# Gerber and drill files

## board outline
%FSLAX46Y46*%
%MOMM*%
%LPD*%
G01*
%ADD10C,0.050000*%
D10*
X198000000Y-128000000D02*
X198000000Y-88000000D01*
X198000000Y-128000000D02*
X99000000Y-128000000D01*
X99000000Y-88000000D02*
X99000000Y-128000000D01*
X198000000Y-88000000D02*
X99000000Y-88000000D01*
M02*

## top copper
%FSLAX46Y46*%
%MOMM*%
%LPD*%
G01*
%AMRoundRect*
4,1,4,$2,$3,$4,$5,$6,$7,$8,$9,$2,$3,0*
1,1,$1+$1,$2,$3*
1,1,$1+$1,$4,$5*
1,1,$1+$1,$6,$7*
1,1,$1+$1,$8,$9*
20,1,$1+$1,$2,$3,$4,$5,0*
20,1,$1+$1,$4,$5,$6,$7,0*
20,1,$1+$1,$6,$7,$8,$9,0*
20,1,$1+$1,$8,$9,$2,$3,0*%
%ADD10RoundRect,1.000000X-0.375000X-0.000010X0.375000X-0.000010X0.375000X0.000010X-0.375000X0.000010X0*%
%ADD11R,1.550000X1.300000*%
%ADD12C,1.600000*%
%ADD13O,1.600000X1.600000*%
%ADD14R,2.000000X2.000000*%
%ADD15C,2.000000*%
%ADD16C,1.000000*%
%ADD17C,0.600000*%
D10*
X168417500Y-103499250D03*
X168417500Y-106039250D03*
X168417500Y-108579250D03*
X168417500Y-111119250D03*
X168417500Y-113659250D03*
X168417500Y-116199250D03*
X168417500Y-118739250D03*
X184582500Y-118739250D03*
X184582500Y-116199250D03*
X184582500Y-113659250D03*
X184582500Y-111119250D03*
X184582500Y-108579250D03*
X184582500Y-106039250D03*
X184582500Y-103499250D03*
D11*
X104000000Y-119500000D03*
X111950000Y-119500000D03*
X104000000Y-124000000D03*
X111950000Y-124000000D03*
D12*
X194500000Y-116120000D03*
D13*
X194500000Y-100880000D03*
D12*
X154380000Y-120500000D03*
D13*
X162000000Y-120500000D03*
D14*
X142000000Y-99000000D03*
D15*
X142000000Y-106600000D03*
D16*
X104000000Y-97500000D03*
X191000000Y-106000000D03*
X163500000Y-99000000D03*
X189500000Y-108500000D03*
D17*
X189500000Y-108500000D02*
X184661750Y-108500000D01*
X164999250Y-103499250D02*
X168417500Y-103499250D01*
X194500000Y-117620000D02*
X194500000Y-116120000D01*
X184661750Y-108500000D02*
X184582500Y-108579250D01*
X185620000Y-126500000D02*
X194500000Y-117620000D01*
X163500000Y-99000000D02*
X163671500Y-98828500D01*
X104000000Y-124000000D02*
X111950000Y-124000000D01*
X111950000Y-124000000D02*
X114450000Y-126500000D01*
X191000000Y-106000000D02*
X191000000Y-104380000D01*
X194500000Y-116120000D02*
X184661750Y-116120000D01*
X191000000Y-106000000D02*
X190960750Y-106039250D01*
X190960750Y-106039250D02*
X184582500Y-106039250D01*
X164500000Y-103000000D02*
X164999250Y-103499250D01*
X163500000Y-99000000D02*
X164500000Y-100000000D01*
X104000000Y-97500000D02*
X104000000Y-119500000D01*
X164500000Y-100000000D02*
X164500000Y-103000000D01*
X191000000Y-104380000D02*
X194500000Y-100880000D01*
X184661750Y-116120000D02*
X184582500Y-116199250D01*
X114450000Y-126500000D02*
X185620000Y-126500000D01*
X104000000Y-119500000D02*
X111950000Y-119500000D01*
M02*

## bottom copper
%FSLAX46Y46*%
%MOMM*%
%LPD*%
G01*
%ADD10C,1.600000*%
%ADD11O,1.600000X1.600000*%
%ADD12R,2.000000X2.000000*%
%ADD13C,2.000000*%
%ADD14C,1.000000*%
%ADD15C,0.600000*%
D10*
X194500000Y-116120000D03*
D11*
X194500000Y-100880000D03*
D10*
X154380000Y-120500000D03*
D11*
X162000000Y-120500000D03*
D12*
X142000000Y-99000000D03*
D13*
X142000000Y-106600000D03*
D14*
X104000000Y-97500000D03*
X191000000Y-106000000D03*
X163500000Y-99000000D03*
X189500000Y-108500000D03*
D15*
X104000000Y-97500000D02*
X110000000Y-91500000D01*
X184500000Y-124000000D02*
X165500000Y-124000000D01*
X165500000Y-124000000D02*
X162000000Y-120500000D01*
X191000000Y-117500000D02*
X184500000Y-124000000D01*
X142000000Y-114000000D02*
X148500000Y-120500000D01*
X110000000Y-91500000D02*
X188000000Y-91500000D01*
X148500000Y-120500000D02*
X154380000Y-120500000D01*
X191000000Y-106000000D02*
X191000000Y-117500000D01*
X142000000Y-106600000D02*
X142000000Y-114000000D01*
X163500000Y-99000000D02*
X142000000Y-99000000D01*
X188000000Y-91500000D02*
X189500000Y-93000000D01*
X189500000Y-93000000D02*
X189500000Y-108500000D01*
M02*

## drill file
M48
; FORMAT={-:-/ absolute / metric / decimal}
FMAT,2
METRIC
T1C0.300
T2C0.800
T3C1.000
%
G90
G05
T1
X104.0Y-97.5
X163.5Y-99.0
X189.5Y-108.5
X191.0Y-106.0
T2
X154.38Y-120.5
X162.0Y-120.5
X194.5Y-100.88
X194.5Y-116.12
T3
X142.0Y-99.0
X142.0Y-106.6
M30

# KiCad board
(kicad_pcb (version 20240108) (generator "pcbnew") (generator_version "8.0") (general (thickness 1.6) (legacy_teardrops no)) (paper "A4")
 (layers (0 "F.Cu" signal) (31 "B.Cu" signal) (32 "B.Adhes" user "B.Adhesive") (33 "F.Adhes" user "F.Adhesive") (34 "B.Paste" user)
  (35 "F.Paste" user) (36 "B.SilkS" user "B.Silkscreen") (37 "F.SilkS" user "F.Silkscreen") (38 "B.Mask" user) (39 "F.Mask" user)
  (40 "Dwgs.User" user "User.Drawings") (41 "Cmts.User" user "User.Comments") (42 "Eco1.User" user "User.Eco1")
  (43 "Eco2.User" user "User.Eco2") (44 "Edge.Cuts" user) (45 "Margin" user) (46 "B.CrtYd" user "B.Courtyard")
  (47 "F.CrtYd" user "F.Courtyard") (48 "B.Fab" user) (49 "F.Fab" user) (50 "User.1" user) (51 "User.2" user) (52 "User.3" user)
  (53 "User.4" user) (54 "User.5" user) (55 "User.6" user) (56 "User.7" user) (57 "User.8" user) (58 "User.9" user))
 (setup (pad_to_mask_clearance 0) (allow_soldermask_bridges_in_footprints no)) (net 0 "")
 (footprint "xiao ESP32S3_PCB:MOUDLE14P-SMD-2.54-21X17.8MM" (layer "F.Cu") (at 167.5825 121.61925)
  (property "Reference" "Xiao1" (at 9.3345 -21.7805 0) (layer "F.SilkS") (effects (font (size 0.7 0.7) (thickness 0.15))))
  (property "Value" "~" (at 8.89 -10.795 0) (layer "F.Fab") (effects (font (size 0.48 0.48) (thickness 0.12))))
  (pad "1" smd roundrect (at 0.835 -18.12) (size 2.75 2) (layers "F.Cu" "F.Paste" "F.Mask") (roundrect_rratio 0.5))
  (pad "2" smd roundrect (at 0.835 -15.58) (size 2.75 2) (layers "F.Cu" "F.Paste" "F.Mask") (roundrect_rratio 0.5))
  (pad "3" smd roundrect (at 0.835 -13.04) (size 2.75 2) (layers "F.Cu" "F.Paste" "F.Mask") (roundrect_rratio 0.5))
  (pad "4" smd roundrect (at 0.835 -10.5) (size 2.75 2) (layers "F.Cu" "F.Paste" "F.Mask") (roundrect_rratio 0.5))
  (pad "5" smd roundrect (at 0.835 -7.96) (size 2.75 2) (layers "F.Cu" "F.Paste" "F.Mask") (roundrect_rratio 0.5))
  (pad "6" smd roundrect (at 0.835 -5.42) (size 2.75 2) (layers "F.Cu" "F.Paste" "F.Mask") (roundrect_rratio 0.5))
  (pad "7" smd roundrect (at 0.835 -2.88) (size 2.75 2) (layers "F.Cu" "F.Paste" "F.Mask") (roundrect_rratio 0.5))
  (pad "8" smd roundrect (at 17 -2.88) (size 2.75 2) (layers "F.Cu" "F.Paste" "F.Mask") (roundrect_rratio 0.5))
  (pad "9" smd roundrect (at 17 -5.42) (size 2.75 2) (layers "F.Cu" "F.Paste" "F.Mask") (roundrect_rratio 0.5))
  (pad "10" smd roundrect (at 17 -7.96) (size 2.75 2) (layers "F.Cu" "F.Paste" "F.Mask") (roundrect_rratio 0.5))
  (pad "11" smd roundrect (at 17 -10.5) (size 2.75 2) (layers "F.Cu" "F.Paste" "F.Mask") (roundrect_rratio 0.5))
  (pad "12" smd roundrect (at 17 -13.04) (size 2.75 2) (layers "F.Cu" "F.Paste" "F.Mask") (roundrect_rratio 0.5))
  (pad "13" smd roundrect (at 17 -15.58) (size 2.75 2) (layers "F.Cu" "F.Paste" "F.Mask") (roundrect_rratio 0.5))
  (pad "14" smd roundrect (at 17 -18.12) (size 2.75 2) (layers "F.Cu" "F.Paste" "F.Mask") (roundrect_rratio 0.5))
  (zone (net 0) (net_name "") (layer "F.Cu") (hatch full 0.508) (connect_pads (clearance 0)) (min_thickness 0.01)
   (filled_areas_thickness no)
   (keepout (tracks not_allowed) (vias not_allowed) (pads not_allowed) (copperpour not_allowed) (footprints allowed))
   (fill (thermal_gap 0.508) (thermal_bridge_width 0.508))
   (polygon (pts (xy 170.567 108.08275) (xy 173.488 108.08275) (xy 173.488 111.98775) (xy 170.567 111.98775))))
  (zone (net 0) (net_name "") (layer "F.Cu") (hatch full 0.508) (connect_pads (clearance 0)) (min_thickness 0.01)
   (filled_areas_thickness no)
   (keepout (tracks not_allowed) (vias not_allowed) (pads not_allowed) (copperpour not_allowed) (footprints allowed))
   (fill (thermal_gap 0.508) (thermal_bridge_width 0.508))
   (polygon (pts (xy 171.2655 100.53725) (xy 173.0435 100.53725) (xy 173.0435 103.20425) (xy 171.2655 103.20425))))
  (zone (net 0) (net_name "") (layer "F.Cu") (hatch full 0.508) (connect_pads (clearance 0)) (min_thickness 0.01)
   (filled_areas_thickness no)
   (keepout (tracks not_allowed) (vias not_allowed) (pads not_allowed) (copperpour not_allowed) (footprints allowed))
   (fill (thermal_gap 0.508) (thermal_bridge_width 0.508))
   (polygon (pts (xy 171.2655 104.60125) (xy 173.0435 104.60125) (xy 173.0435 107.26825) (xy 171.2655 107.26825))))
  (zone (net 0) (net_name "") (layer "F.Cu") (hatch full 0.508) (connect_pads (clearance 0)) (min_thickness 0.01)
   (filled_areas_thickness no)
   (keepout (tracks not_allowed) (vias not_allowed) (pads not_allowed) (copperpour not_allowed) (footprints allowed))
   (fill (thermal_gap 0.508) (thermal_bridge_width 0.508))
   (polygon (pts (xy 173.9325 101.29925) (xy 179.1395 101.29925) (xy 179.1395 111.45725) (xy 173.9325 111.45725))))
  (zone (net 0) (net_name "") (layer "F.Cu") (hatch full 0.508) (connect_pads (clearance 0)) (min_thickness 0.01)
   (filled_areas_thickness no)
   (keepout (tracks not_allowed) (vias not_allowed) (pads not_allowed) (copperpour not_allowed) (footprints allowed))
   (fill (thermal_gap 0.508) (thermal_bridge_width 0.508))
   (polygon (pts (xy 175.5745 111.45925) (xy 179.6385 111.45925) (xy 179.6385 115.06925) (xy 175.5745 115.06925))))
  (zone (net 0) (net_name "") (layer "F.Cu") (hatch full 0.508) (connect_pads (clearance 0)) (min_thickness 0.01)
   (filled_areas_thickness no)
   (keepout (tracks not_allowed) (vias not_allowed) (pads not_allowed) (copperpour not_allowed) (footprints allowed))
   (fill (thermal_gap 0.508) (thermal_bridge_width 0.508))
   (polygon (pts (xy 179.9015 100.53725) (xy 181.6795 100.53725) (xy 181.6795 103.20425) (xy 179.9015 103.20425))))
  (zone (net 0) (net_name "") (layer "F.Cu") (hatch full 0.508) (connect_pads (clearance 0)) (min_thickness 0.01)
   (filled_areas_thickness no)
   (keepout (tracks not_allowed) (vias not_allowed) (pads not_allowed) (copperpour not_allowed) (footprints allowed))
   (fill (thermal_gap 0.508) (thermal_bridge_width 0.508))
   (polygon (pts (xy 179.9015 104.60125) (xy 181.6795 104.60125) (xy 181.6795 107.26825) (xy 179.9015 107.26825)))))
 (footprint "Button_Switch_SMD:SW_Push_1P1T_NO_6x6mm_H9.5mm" (layer "F.Cu") (at 107.975 121.75)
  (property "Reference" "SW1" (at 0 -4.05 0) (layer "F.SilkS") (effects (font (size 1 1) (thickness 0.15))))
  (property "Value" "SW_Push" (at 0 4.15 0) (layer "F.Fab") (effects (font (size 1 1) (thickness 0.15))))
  (pad "1" smd rect (at -3.975 -2.25) (size 1.55 1.3) (layers "F.Cu" "F.Paste" "F.Mask"))
  (pad "1" smd rect (at 3.975 -2.25) (size 1.55 1.3) (layers "F.Cu" "F.Paste" "F.Mask"))
  (pad "2" smd rect (at -3.975 2.25) (size 1.55 1.3) (layers "F.Cu" "F.Paste" "F.Mask"))
  (pad "2" smd rect (at 3.975 2.25) (size 1.55 1.3) (layers "F.Cu" "F.Paste" "F.Mask")))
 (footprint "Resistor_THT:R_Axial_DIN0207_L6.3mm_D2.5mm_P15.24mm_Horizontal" (layer "F.Cu") (at 194.5 116.12 90)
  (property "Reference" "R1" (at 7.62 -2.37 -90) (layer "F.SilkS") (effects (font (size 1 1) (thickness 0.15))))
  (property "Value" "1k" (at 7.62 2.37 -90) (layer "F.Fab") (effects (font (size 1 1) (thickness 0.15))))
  (pad "1" thru_hole circle (at 0 0 90) (size 1.6 1.6) (drill 0.8) (layers "*.Cu" "*.Mask") (remove_unused_layers no))
  (pad "2" thru_hole oval (at 15.24 0 90) (size 1.6 1.6) (drill 0.8) (layers "*.Cu" "*.Mask") (remove_unused_layers no)))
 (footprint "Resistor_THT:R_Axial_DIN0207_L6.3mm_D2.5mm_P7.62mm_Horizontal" (layer "F.Cu") (at 154.38 120.5)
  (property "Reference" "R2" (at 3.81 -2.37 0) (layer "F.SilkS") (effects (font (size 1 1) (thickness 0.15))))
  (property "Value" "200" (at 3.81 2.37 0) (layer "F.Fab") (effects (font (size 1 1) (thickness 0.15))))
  (pad "1" thru_hole circle (at 0 0) (size 1.6 1.6) (drill 0.8) (layers "*.Cu" "*.Mask") (remove_unused_layers no))
  (pad "2" thru_hole oval (at 7.62 0) (size 1.6 1.6) (drill 0.8) (layers "*.Cu" "*.Mask") (remove_unused_layers no)))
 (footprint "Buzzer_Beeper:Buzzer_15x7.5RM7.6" (layer "F.Cu") (at 142 99 -90)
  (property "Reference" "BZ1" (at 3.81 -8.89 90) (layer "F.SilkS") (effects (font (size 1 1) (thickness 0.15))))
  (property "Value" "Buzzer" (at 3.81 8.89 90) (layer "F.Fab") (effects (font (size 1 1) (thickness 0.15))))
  (pad "1" thru_hole rect (at 0 0 270) (size 2 2) (drill 1) (layers "*.Cu" "*.Mask") (remove_unused_layers no))
  (pad "2" thru_hole circle (at 7.6 0 270) (size 2 2) (drill 1) (layers "*.Cu" "*.Mask") (remove_unused_layers no)))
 (gr_line (start 198 128) (end 198 88) (stroke (width 0.05) (type default)) (layer "Edge.Cuts"))
 (gr_line (start 198 128) (end 99 128) (stroke (width 0.05) (type default)) (layer "Edge.Cuts"))
 (gr_line (start 99 88) (end 99 128) (stroke (width 0.05) (type default)) (layer "Edge.Cuts"))
 (gr_line (start 198 88) (end 99 88) (stroke (width 0.05) (type default)) (layer "Edge.Cuts"))
 (segment (start 189.5 108.5) (end 184.66175 108.5) (width 0.6) (layer "F.Cu") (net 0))
 (segment (start 164.99925 103.49925) (end 168.4175 103.49925) (width 0.6) (layer "F.Cu") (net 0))
 (segment (start 194.5 117.62) (end 194.5 116.12) (width 0.6) (layer "F.Cu") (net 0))
 (segment (start 184.66175 108.5) (end 184.5825 108.57925) (width 0.6) (layer "F.Cu") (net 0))
 (segment (start 185.62 126.5) (end 194.5 117.62) (width 0.6) (layer "F.Cu") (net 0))
 (segment (start 163.5 99) (end 163.6715 98.8285) (width 0.6) (layer "F.Cu") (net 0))
 (segment (start 104 124) (end 111.95 124) (width 0.6) (layer "F.Cu") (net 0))
 (segment (start 111.95 124) (end 114.45 126.5) (width 0.6) (layer "F.Cu") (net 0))
 (segment (start 191 106) (end 191 104.38) (width 0.6) (layer "F.Cu") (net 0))
 (segment (start 194.5 116.12) (end 184.66175 116.12) (width 0.6) (layer "F.Cu") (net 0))
 (segment (start 191 106) (end 190.96075 106.03925) (width 0.6) (layer "F.Cu") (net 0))
 (segment (start 190.96075 106.03925) (end 184.5825 106.03925) (width 0.6) (layer "F.Cu") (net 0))
 (segment (start 164.5 103) (end 164.99925 103.49925) (width 0.6) (layer "F.Cu") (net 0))
 (segment (start 163.5 99) (end 164.5 100) (width 0.6) (layer "F.Cu") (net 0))
 (segment (start 104 97.5) (end 104 119.5) (width 0.6) (layer "F.Cu") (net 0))
 (segment (start 164.5 100) (end 164.5 103) (width 0.6) (layer "F.Cu") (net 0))
 (segment (start 191 104.38) (end 194.5 100.88) (width 0.6) (layer "F.Cu") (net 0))
 (segment (start 184.66175 116.12) (end 184.5825 116.19925) (width 0.6) (layer "F.Cu") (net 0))
 (segment (start 114.45 126.5) (end 185.62 126.5) (width 0.6) (layer "F.Cu") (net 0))
 (segment (start 104 119.5) (end 111.95 119.5) (width 0.6) (layer "F.Cu") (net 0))
 (via (at 104 97.5) (size 1) (drill 0.3) (layers "F.Cu" "B.Cu") (free yes) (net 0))
 (via (at 191 106) (size 1) (drill 0.3) (layers "F.Cu" "B.Cu") (free yes) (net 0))
 (via (at 163.5 99) (size 1) (drill 0.3) (layers "F.Cu" "B.Cu") (free yes) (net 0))
 (via (at 189.5 108.5) (size 1) (drill 0.3) (layers "F.Cu" "B.Cu") (free yes) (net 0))
 (segment (start 104 97.5) (end 110 91.5) (width 0.6) (layer "B.Cu") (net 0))
 (segment (start 184.5 124) (end 165.5 124) (width 0.6) (layer "B.Cu") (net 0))
 (segment (start 165.5 124) (end 162 120.5) (width 0.6) (layer "B.Cu") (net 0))
 (segment (start 191 117.5) (end 184.5 124) (width 0.6) (layer "B.Cu") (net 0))
 (segment (start 142 114) (end 148.5 120.5) (width 0.6) (layer "B.Cu") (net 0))
 (segment (start 110 91.5) (end 188 91.5) (width 0.6) (layer "B.Cu") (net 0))
 (segment (start 148.5 120.5) (end 154.38 120.5) (width 0.6) (layer "B.Cu") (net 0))
 (segment (start 191 106) (end 191 117.5) (width 0.6) (layer "B.Cu") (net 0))
 (segment (start 142 106.6) (end 142 114) (width 0.6) (layer "B.Cu") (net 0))
 (segment (start 163.5 99) (end 142 99) (width 0.6) (layer "B.Cu") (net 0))
 (segment (start 188 91.5) (end 189.5 93) (width 0.6) (layer "B.Cu") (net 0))
 (segment (start 189.5 93) (end 189.5 108.5) (width 0.6) (layer "B.Cu") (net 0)))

